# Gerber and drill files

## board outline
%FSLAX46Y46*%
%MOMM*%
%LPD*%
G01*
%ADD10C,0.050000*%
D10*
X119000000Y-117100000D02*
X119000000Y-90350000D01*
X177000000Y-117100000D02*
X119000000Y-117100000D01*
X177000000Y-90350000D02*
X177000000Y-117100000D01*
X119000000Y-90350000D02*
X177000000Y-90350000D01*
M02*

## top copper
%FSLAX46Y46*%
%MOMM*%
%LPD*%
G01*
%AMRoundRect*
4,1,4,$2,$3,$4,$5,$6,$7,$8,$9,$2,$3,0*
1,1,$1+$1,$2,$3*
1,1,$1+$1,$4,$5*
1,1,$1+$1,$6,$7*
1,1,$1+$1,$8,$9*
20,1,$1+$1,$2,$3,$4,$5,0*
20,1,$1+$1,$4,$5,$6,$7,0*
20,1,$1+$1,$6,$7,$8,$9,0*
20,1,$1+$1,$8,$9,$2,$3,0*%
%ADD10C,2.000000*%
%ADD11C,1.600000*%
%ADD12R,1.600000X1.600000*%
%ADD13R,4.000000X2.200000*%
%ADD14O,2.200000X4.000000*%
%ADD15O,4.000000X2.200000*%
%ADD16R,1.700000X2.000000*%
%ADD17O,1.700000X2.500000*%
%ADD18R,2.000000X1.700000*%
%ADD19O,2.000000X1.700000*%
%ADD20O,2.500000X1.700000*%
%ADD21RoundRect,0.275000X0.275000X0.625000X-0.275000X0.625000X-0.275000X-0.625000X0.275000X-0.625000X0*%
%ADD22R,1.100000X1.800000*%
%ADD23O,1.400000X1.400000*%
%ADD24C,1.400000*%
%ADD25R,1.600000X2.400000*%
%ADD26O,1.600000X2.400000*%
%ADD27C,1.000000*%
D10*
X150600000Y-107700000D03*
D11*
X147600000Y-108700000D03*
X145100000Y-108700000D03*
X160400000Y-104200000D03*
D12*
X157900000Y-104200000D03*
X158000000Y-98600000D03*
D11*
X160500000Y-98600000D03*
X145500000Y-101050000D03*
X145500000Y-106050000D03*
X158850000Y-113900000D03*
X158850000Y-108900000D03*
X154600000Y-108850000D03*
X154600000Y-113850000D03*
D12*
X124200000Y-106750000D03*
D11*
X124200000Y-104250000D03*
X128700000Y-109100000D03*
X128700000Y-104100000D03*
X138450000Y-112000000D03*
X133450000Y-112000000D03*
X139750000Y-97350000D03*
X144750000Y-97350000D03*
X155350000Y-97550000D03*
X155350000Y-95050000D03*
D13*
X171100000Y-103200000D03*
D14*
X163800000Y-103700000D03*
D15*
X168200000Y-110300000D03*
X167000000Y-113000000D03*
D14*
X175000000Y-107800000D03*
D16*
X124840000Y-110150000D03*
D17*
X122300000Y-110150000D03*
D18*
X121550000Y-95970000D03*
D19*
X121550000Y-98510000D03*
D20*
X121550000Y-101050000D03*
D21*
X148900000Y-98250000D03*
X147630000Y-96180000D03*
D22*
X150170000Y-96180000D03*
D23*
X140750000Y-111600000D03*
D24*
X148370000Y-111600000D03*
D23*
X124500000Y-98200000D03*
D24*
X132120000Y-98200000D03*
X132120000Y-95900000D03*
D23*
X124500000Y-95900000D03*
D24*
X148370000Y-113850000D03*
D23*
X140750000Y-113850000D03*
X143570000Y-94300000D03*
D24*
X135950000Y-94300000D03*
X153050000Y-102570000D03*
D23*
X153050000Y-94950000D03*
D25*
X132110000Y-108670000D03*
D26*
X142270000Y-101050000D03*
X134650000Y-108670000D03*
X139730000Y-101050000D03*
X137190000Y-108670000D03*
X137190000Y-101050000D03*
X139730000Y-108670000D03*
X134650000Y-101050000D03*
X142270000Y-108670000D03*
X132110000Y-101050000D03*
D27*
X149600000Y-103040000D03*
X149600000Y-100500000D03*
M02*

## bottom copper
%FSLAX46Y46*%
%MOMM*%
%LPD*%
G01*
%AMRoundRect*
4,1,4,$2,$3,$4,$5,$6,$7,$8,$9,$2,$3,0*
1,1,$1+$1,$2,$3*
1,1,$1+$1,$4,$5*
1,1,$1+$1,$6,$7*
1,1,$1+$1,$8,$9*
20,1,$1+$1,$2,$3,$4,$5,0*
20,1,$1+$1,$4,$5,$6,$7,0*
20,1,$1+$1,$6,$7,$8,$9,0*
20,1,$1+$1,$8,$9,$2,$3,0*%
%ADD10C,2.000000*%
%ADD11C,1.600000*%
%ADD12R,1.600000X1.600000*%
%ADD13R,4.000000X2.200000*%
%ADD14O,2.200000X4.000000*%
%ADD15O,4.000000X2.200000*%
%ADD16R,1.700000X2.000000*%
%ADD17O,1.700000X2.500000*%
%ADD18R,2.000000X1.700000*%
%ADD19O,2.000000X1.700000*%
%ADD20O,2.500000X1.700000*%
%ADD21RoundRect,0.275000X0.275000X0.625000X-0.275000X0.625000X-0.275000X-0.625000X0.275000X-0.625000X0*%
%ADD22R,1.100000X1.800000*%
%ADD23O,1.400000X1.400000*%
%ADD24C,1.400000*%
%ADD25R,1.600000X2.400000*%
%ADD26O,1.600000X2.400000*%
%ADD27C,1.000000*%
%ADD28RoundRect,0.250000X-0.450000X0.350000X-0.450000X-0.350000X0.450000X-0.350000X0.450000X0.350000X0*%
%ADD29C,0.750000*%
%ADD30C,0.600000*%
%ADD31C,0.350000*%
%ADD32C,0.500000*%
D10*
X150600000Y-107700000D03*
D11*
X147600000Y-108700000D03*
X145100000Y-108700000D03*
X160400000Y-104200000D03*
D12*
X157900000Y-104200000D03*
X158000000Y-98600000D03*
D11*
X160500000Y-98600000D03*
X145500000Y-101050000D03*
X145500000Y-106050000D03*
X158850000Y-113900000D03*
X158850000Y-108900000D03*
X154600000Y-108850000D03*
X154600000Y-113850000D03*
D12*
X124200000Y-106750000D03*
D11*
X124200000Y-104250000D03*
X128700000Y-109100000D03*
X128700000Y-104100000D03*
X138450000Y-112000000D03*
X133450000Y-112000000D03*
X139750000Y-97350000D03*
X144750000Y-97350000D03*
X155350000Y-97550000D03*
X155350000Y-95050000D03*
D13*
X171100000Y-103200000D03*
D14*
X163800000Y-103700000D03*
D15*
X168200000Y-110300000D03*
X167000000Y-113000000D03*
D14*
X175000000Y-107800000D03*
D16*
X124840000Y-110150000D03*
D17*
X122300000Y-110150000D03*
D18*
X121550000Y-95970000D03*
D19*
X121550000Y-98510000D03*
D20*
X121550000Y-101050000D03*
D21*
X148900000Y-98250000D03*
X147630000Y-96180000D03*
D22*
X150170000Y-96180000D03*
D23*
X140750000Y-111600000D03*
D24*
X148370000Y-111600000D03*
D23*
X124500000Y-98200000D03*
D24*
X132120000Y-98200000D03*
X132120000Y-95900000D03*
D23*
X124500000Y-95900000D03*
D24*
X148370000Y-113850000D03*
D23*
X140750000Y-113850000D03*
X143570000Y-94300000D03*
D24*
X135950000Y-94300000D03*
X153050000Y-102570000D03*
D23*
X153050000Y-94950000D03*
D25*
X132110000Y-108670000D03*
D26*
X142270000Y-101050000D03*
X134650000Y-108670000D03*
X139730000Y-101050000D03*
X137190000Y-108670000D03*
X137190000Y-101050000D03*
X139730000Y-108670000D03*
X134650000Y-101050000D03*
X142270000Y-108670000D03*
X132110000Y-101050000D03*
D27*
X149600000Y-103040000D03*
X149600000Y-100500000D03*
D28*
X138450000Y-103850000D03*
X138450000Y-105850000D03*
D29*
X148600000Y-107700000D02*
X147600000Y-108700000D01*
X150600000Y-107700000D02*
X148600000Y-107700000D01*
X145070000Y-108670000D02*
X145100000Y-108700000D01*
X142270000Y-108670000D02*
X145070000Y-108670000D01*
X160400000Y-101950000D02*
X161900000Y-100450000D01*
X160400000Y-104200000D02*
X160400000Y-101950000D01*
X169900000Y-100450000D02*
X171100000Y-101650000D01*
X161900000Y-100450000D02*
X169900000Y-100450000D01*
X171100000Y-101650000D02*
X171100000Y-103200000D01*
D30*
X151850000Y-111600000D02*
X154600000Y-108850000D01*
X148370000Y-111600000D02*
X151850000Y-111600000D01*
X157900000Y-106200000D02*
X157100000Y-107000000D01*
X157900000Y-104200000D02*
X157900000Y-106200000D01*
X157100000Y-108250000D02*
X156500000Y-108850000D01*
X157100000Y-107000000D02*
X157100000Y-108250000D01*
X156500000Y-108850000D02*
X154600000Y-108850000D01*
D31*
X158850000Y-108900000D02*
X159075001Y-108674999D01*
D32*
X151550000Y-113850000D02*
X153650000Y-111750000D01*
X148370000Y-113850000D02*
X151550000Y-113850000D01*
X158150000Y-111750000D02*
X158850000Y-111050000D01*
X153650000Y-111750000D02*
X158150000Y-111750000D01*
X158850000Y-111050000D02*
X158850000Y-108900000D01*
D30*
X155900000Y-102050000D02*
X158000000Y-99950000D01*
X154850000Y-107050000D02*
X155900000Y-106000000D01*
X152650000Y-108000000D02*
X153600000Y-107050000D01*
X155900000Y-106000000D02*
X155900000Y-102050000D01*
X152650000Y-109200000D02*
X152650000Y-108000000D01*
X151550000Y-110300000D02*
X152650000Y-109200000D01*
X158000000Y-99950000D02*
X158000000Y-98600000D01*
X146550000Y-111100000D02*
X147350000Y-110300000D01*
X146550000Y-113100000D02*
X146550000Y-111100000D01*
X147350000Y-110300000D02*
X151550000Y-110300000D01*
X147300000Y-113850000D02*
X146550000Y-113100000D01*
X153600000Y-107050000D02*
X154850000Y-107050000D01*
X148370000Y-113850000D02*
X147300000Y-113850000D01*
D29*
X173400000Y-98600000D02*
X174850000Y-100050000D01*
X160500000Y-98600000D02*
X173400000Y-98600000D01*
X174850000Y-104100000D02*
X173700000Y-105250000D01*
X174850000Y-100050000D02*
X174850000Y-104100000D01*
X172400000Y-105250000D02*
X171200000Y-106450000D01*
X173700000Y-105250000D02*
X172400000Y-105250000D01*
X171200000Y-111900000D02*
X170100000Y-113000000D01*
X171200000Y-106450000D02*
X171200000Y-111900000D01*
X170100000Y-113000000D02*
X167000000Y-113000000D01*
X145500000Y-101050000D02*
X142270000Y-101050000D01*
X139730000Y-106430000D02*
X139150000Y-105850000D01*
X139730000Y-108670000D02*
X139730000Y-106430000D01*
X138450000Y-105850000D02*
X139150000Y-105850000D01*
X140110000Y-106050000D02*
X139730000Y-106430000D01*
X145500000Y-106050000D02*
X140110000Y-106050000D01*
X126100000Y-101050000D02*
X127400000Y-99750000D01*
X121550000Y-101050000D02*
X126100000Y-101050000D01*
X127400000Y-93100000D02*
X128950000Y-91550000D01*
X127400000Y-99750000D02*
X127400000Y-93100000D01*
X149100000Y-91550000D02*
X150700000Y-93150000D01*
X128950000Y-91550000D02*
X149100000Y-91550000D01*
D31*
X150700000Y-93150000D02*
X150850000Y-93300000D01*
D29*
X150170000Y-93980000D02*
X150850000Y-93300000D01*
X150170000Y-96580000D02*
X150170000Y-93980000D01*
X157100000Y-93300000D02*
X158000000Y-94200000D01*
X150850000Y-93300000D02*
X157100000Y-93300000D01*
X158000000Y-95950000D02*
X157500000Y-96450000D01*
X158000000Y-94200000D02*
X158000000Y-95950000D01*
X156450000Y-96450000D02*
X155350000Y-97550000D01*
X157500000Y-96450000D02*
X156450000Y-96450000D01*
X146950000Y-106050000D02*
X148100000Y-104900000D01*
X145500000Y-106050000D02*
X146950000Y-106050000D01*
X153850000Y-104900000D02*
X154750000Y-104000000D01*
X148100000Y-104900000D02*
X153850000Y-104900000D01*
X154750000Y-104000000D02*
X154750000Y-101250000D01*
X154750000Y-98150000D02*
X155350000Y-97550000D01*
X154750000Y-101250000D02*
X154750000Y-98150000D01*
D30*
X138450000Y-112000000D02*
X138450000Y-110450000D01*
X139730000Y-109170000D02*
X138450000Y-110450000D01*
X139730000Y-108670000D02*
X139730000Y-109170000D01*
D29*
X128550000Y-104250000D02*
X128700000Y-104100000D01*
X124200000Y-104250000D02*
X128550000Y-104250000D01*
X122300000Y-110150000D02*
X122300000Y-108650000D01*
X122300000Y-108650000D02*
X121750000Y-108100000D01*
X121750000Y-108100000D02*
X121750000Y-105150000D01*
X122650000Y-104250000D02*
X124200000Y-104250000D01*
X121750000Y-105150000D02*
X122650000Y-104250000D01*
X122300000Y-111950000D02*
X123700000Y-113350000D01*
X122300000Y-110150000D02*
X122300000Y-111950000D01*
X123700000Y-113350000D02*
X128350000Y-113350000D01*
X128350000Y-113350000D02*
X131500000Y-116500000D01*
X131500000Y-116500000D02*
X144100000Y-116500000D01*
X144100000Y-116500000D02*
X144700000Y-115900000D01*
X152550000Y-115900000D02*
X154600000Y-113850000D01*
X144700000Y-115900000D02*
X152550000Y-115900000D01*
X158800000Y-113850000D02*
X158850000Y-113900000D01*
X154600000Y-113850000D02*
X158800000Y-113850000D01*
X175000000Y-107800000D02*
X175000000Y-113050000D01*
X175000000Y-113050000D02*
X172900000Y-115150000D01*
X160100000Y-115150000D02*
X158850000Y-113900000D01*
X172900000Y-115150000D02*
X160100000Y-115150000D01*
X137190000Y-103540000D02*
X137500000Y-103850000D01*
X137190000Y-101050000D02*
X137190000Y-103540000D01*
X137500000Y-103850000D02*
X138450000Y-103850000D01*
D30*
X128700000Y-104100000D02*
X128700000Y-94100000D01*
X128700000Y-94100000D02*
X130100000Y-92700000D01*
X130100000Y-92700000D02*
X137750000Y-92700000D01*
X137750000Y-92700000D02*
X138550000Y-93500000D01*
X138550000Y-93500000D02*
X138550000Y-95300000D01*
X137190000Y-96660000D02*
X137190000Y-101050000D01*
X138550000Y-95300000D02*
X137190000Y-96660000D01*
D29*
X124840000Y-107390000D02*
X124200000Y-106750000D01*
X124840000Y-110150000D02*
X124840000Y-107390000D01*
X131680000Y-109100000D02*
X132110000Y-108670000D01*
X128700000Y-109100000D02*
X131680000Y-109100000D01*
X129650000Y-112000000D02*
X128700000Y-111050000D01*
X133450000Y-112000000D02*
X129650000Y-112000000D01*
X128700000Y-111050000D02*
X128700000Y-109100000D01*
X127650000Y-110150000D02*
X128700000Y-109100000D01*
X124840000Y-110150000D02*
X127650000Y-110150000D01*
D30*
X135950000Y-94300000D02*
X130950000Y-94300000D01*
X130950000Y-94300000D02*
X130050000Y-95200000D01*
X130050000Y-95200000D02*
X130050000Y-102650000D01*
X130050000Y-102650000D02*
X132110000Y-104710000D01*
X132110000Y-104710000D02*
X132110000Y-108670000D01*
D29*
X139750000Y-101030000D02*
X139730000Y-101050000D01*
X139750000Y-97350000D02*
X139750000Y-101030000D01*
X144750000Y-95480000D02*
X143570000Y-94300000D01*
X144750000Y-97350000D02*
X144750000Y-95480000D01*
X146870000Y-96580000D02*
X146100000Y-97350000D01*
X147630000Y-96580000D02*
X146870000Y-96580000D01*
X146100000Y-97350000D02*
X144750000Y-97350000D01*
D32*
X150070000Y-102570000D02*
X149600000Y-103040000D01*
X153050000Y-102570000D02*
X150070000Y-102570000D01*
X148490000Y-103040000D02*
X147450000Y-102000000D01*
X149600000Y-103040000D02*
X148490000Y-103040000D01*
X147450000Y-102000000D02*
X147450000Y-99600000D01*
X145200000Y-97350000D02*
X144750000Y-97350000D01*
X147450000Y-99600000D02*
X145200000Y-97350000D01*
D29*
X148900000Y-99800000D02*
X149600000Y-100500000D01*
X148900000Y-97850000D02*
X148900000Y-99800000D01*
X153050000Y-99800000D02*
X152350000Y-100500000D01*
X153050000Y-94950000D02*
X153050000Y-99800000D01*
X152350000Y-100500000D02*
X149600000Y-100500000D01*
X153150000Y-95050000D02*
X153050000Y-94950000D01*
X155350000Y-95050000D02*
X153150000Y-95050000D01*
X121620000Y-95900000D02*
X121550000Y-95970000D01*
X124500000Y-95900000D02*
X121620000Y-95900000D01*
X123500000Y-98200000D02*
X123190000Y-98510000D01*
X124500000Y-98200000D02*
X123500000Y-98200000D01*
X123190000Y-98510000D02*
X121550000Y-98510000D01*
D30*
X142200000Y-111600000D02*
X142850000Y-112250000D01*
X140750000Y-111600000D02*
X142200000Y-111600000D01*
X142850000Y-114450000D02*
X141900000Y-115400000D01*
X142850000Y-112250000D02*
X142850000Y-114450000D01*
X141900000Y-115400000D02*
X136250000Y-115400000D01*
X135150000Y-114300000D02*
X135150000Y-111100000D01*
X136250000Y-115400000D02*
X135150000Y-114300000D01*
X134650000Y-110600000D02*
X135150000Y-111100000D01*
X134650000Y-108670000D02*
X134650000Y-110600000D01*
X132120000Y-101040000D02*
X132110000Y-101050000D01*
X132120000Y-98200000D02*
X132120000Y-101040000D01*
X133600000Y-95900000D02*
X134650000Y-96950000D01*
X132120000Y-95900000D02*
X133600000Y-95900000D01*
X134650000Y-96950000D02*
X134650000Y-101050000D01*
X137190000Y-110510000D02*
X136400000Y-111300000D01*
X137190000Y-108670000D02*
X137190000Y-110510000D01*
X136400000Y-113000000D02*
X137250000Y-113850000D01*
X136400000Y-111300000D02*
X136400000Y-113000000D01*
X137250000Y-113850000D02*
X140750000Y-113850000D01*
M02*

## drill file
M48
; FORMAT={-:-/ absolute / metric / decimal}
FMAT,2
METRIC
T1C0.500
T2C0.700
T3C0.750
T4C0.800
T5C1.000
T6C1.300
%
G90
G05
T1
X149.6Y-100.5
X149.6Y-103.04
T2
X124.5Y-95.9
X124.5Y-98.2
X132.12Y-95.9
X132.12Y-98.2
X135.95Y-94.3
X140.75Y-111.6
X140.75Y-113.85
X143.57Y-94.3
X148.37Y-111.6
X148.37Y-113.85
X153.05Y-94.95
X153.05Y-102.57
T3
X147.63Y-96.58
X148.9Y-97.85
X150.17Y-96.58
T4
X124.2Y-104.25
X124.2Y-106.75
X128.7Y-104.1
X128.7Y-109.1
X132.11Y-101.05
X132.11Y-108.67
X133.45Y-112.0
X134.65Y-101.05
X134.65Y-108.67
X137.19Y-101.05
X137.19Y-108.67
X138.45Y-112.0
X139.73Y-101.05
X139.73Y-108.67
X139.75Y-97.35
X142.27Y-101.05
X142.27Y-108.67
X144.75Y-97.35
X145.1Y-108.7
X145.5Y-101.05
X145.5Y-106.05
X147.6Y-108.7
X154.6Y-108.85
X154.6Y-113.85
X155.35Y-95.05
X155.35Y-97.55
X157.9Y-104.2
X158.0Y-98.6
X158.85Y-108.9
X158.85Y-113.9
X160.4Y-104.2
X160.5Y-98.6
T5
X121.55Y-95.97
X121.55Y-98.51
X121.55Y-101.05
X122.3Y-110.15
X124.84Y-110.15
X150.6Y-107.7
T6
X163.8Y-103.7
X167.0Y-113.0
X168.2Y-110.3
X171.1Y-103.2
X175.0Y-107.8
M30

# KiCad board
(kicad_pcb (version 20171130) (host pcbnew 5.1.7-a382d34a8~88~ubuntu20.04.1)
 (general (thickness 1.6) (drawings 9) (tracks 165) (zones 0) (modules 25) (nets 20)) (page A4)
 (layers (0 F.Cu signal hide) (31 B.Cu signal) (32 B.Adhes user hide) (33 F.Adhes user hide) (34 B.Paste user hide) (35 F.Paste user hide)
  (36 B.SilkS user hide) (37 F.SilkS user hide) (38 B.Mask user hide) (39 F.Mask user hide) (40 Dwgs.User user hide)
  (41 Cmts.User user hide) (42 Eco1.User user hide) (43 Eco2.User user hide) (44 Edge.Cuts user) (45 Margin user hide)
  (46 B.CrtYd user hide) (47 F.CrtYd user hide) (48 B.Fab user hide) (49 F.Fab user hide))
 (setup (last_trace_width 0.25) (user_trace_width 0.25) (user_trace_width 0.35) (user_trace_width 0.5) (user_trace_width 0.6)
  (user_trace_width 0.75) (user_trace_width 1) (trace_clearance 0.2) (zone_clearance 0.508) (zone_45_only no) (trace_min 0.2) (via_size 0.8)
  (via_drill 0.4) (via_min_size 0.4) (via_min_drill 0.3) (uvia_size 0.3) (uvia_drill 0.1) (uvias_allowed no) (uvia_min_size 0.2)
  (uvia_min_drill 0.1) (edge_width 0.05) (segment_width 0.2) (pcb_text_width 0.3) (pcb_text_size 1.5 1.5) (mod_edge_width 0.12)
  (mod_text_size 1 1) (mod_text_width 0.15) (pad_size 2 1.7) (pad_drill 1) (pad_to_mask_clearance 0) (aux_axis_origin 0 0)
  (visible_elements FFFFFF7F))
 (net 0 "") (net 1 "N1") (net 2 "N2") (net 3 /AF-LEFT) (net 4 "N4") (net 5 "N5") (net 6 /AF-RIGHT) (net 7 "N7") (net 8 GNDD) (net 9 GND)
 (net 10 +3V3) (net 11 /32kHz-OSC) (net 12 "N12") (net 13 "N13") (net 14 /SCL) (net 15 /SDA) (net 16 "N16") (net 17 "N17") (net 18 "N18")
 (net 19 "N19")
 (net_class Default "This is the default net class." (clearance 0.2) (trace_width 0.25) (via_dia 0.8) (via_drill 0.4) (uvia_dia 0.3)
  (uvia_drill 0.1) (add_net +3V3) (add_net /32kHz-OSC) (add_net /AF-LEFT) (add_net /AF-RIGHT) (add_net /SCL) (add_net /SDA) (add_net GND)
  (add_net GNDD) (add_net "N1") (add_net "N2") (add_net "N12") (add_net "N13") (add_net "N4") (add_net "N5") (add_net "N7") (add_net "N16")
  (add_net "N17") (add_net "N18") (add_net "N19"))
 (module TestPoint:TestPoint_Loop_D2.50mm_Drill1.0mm (layer F.Cu) (at 150.6 107.7)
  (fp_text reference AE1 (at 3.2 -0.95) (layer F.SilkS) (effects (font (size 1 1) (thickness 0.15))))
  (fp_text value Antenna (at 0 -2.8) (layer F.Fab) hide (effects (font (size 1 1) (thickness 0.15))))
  (pad 1 thru_hole circle (at 0 0) (size 2 2) (drill 1) (layers *.Cu *.Mask) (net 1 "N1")))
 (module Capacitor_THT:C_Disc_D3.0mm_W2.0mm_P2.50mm (layer F.Cu) (at 147.6 108.7 180)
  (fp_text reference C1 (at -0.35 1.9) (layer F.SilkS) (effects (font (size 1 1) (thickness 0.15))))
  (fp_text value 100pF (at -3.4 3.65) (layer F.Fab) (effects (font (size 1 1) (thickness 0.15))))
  (pad 1 thru_hole circle (at 0 0 180) (size 1.6 1.6) (drill 0.8) (layers *.Cu *.Mask) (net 1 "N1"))
  (pad 2 thru_hole circle (at 2.5 0 180) (size 1.6 1.6) (drill 0.8) (layers *.Cu *.Mask) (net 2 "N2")))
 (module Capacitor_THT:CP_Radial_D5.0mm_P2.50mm (layer F.Cu) (at 157.9 104.2)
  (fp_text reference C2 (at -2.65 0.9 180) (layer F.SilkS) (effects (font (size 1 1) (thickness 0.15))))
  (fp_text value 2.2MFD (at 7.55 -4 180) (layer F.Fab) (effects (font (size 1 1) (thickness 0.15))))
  (pad 2 thru_hole circle (at 2.5 0) (size 1.6 1.6) (drill 0.8) (layers *.Cu *.Mask) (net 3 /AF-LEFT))
  (pad 1 thru_hole rect (at 0 0) (size 1.6 1.6) (drill 0.8) (layers *.Cu *.Mask) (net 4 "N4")))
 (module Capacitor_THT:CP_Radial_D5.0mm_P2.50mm (layer F.Cu) (at 158 98.6)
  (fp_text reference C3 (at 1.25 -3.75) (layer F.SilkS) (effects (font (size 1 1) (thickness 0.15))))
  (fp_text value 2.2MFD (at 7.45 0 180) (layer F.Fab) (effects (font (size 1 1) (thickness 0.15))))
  (pad 1 thru_hole rect (at 0 0) (size 1.6 1.6) (drill 0.8) (layers *.Cu *.Mask) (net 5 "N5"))
  (pad 2 thru_hole circle (at 2.5 0) (size 1.6 1.6) (drill 0.8) (layers *.Cu *.Mask) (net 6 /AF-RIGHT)))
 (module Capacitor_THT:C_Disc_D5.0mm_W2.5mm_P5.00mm (layer F.Cu) (at 145.5 101.05 270)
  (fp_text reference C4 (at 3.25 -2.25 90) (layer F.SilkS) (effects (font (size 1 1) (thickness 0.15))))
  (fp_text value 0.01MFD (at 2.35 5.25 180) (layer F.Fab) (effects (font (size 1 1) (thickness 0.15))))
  (pad 1 thru_hole circle (at 0 0 270) (size 1.6 1.6) (drill 0.8) (layers *.Cu *.Mask) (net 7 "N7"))
  (pad 2 thru_hole circle (at 5 0 270) (size 1.6 1.6) (drill 0.8) (layers *.Cu *.Mask) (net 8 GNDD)))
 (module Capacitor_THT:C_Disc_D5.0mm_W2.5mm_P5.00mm (layer F.Cu) (at 158.85 108.9 270)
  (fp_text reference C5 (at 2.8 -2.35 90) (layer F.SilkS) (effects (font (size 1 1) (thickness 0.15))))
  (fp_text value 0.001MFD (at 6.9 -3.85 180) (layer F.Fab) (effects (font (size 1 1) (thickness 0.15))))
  (pad 2 thru_hole circle (at 5 0 270) (size 1.6 1.6) (drill 0.8) (layers *.Cu *.Mask) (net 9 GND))
  (pad 1 thru_hole circle (at 0 0 270) (size 1.6 1.6) (drill 0.8) (layers *.Cu *.Mask) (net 5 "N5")))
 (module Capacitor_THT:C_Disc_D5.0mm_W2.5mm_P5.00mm (layer F.Cu) (at 154.6 108.85 270)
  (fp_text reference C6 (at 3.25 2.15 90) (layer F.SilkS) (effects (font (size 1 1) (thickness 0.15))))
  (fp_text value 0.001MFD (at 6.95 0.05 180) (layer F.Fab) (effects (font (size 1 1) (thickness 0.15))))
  (pad 1 thru_hole circle (at 0 0 270) (size 1.6 1.6) (drill 0.8) (layers *.Cu *.Mask) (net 4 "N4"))
  (pad 2 thru_hole circle (at 5 0 270) (size 1.6 1.6) (drill 0.8) (layers *.Cu *.Mask) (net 9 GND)))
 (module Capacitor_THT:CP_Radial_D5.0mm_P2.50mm (layer F.Cu) (at 124.2 106.75 90)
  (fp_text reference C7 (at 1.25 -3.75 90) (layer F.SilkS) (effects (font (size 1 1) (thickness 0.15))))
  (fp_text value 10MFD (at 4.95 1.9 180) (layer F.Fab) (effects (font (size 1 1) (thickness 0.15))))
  (pad 1 thru_hole rect (at 0 0 90) (size 1.6 1.6) (drill 0.8) (layers *.Cu *.Mask) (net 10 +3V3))
  (pad 2 thru_hole circle (at 2.5 0 90) (size 1.6 1.6) (drill 0.8) (layers *.Cu *.Mask) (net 9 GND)))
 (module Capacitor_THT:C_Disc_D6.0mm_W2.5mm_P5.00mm (layer F.Cu) (at 128.7 109.1 90)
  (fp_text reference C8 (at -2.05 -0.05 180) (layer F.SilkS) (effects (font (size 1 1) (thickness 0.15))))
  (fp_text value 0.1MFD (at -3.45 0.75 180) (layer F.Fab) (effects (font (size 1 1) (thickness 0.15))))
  (pad 1 thru_hole circle (at 0 0 90) (size 1.6 1.6) (drill 0.8) (layers *.Cu *.Mask) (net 10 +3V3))
  (pad 2 thru_hole circle (at 5 0 90) (size 1.6 1.6) (drill 0.8) (layers *.Cu *.Mask) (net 9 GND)))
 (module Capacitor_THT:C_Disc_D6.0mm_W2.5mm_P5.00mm (layer F.Cu) (at 133.45 112)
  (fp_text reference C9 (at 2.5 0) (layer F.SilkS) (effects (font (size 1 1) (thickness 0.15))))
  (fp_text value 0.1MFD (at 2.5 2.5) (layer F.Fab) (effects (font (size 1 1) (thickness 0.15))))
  (pad 2 thru_hole circle (at 5 0) (size 1.6 1.6) (drill 0.8) (layers *.Cu *.Mask) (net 8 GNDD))
  (pad 1 thru_hole circle (at 0 0) (size 1.6 1.6) (drill 0.8) (layers *.Cu *.Mask) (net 10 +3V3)))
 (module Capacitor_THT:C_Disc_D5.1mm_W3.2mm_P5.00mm (layer F.Cu) (at 139.75 97.35)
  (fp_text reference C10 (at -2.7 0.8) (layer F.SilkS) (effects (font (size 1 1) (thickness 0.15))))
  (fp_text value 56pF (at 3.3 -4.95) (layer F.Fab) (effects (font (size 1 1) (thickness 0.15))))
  (pad 1 thru_hole circle (at 0 0) (size 1.6 1.6) (drill 0.8) (layers *.Cu *.Mask) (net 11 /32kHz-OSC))
  (pad 2 thru_hole circle (at 5 0) (size 1.6 1.6) (drill 0.8) (layers *.Cu *.Mask) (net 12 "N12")))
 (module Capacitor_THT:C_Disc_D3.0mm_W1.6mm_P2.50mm (layer F.Cu) (at 155.35 97.55 90)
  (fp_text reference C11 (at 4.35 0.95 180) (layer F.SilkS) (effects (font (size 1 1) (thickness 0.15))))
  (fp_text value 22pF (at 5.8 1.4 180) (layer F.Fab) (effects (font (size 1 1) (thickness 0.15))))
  (pad 1 thru_hole circle (at 0 0 90) (size 1.6 1.6) (drill 0.8) (layers *.Cu *.Mask) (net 8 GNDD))
  (pad 2 thru_hole circle (at 2.5 0 90) (size 1.6 1.6) (drill 0.8) (layers *.Cu *.Mask) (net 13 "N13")))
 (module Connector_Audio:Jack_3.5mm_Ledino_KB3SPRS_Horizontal (layer F.Cu) (at 171.1 103.2 180)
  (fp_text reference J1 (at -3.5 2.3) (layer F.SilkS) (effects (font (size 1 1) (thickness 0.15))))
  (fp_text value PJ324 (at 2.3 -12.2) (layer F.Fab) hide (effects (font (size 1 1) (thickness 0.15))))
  (pad T thru_hole rect (at 0 0 180) (size 4 2.2) (drill 1.3) (layers *.Cu *.Mask) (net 3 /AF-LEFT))
  (pad TN thru_hole oval (at 7.3 -0.5 270) (size 4 2.2) (drill 1.3) (layers *.Cu *.Mask))
  (pad RN thru_hole oval (at 2.9 -7.1 180) (size 4 2.2) (drill 1.3) (layers *.Cu *.Mask))
  (pad R thru_hole oval (at 4.1 -9.8 180) (size 4 2.2) (drill 1.3) (layers *.Cu *.Mask) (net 6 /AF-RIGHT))
  (pad S thru_hole oval (at -3.9 -4.6 180) (size 2.2 4) (drill 1.3) (layers *.Cu *.Mask) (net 9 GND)))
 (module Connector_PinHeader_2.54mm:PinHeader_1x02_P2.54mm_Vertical (layer F.Cu) (at 124.84 110.15 270)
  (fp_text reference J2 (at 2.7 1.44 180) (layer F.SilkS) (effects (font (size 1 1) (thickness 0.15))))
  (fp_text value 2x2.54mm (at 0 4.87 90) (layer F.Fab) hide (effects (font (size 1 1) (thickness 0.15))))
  (pad 1 thru_hole rect (at 0 0 270) (size 2 1.7) (drill 1) (layers *.Cu *.Mask) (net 10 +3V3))
  (pad 2 thru_hole oval (at 0 2.54 270) (size 2.5 1.7) (drill 1) (layers *.Cu *.Mask) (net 9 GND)))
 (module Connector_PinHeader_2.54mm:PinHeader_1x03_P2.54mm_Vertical (layer F.Cu) (at 121.55 95.97)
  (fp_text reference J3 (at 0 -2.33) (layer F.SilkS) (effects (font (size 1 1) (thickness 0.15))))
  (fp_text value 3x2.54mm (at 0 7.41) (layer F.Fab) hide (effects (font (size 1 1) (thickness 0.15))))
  (pad 1 thru_hole rect (at 0 0) (size 2 1.7) (drill 1) (layers *.Cu *.Mask) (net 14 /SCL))
  (pad 2 thru_hole oval (at 0 2.54) (size 2 1.7) (drill 1) (layers *.Cu *.Mask) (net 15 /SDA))
  (pad 3 thru_hole oval (at 0 5.08) (size 2.5 1.7) (drill 1) (layers *.Cu *.Mask) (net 8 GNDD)))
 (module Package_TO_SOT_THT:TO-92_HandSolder (layer F.Cu) (at 150.17 96.58 180)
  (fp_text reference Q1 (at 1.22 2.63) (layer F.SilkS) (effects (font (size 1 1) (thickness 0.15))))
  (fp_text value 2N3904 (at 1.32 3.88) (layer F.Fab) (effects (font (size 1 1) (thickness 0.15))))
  (pad 2 thru_hole roundrect (at 1.27 -1.27 180) (size 1.1 1.8) (drill 0.75 (offset 0 -0.4)) (layers *.Cu *.Mask) (roundrect_rratio 0.25)
   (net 13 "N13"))
  (pad 3 thru_hole roundrect (at 2.54 0 180) (size 1.1 1.8) (drill 0.75 (offset 0 0.4)) (layers *.Cu *.Mask) (roundrect_rratio 0.25)
   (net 12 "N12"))
  (pad 1 thru_hole rect (at 0 0 180) (size 1.1 1.8) (drill 0.75 (offset 0 0.4)) (layers *.Cu *.Mask) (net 8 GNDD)))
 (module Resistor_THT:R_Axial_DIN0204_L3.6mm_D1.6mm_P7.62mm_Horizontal (layer F.Cu) (at 148.37 111.6 180)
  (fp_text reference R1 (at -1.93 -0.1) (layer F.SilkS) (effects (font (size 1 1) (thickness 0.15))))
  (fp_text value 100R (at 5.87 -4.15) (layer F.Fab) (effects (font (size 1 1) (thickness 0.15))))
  (pad 2 thru_hole oval (at 7.62 0 180) (size 1.4 1.4) (drill 0.7) (layers *.Cu *.Mask) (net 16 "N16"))
  (pad 1 thru_hole circle (at 0 0 180) (size 1.4 1.4) (drill 0.7) (layers *.Cu *.Mask) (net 4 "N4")))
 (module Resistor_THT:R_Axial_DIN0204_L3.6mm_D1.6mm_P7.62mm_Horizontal (layer F.Cu) (at 132.12 98.2 180)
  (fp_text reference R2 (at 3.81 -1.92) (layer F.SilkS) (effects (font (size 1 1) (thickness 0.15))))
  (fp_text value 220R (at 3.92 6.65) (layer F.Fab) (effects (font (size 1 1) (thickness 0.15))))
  (pad 2 thru_hole oval (at 7.62 0 180) (size 1.4 1.4) (drill 0.7) (layers *.Cu *.Mask) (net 15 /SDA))
  (pad 1 thru_hole circle (at 0 0 180) (size 1.4 1.4) (drill 0.7) (layers *.Cu *.Mask) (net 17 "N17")))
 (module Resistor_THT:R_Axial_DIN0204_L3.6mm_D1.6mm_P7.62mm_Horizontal (layer F.Cu) (at 132.12 95.9 180)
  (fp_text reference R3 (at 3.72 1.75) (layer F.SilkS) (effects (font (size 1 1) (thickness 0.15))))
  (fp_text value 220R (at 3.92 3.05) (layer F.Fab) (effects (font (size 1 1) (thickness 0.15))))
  (pad 1 thru_hole circle (at 0 0 180) (size 1.4 1.4) (drill 0.7) (layers *.Cu *.Mask) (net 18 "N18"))
  (pad 2 thru_hole oval (at 7.62 0 180) (size 1.4 1.4) (drill 0.7) (layers *.Cu *.Mask) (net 14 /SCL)))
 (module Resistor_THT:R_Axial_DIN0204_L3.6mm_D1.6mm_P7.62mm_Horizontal (layer F.Cu) (at 148.37 113.85 180)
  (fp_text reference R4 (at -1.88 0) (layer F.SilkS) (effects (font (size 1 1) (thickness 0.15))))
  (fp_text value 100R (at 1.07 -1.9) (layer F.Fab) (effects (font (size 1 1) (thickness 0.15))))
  (pad 1 thru_hole circle (at 0 0 180) (size 1.4 1.4) (drill 0.7) (layers *.Cu *.Mask) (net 5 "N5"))
  (pad 2 thru_hole oval (at 7.62 0 180) (size 1.4 1.4) (drill 0.7) (layers *.Cu *.Mask) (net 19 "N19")))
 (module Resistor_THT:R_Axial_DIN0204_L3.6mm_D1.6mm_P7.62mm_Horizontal (layer F.Cu) (at 135.95 94.3)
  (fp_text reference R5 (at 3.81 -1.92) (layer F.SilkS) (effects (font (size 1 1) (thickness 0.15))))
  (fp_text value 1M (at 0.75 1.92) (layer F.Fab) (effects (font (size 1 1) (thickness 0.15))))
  (pad 2 thru_hole oval (at 7.62 0) (size 1.4 1.4) (drill 0.7) (layers *.Cu *.Mask) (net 12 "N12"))
  (pad 1 thru_hole circle (at 0 0) (size 1.4 1.4) (drill 0.7) (layers *.Cu *.Mask) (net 10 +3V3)))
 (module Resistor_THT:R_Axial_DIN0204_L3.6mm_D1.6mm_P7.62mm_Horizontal (layer F.Cu) (at 153.05 102.57 90)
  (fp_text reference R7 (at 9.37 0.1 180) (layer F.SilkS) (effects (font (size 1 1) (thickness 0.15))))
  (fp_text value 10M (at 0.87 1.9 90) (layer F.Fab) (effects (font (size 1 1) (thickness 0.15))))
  (pad 1 thru_hole circle (at 0 0 90) (size 1.4 1.4) (drill 0.7) (layers *.Cu *.Mask) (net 12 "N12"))
  (pad 2 thru_hole oval (at 7.62 0 90) (size 1.4 1.4) (drill 0.7) (layers *.Cu *.Mask) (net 13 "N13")))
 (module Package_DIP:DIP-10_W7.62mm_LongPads (layer F.Cu) (at 132.11 108.67 90)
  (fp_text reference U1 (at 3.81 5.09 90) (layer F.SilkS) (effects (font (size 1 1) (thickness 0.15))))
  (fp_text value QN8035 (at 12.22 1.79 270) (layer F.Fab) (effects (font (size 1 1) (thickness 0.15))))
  (pad 1 thru_hole rect (at 0 0 90) (size 2.4 1.6) (drill 0.8) (layers *.Cu *.Mask) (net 10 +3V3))
  (pad 6 thru_hole oval (at 7.62 10.16 90) (size 2.4 1.6) (drill 0.8) (layers *.Cu *.Mask) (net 7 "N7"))
  (pad 2 thru_hole oval (at 0 2.54 90) (size 2.4 1.6) (drill 0.8) (layers *.Cu *.Mask) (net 16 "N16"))
  (pad 7 thru_hole oval (at 7.62 7.62 90) (size 2.4 1.6) (drill 0.8) (layers *.Cu *.Mask) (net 11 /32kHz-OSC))
  (pad 3 thru_hole oval (at 0 5.08 90) (size 2.4 1.6) (drill 0.8) (layers *.Cu *.Mask) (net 19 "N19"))
  (pad 8 thru_hole oval (at 7.62 5.08 90) (size 2.4 1.6) (drill 0.8) (layers *.Cu *.Mask) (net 9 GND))
  (pad 4 thru_hole oval (at 0 7.62 90) (size 2.4 1.6) (drill 0.8) (layers *.Cu *.Mask) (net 8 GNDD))
  (pad 9 thru_hole oval (at 7.62 2.54 90) (size 2.4 1.6) (drill 0.8) (layers *.Cu *.Mask) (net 18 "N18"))
  (pad 5 thru_hole oval (at 0 10.16 90) (size 2.4 1.6) (drill 0.8) (layers *.Cu *.Mask) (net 2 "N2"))
  (pad 10 thru_hole oval (at 7.62 0 90) (size 2.4 1.6) (drill 0.8) (layers *.Cu *.Mask) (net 17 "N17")))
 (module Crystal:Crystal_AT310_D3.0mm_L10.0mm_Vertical (layer F.Cu) (at 149.6 103.04 90)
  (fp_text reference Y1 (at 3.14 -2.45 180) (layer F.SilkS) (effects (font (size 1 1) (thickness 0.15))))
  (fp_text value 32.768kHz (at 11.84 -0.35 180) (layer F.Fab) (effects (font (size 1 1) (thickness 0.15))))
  (pad 1 thru_hole circle (at 0 0 90) (size 1 1) (drill 0.5) (layers *.Cu *.Mask) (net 12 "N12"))
  (pad 2 thru_hole circle (at 2.54 0 90) (size 1 1) (drill 0.5) (layers *.Cu *.Mask) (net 13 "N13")))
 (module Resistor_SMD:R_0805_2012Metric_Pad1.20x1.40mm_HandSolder (layer B.Cu) (at 138.45 104.85 270)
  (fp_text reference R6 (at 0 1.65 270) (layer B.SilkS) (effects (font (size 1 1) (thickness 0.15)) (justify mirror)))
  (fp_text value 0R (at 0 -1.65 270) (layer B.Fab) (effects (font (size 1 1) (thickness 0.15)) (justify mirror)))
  (pad 1 smd roundrect (at -1 0 270) (size 1.2 1.4) (layers B.Cu B.Paste B.Mask) (roundrect_rratio 0.208333) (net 9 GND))
  (pad 2 smd roundrect (at 1 0 270) (size 1.2 1.4) (layers B.Cu B.Paste B.Mask) (roundrect_rratio 0.208333) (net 8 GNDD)))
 (gr_line (start 119 117.1) (end 119 90.35) (layer Edge.Cuts) (width 0.05))
 (gr_line (start 177 117.1) (end 119 117.1) (layer Edge.Cuts) (width 0.05))
 (gr_line (start 177 90.35) (end 177 117.1) (layer Edge.Cuts) (width 0.05))
 (gr_line (start 119 90.35) (end 177 90.35) (layer Edge.Cuts) (width 0.05))
 (segment (start 148.6 107.7) (end 147.6 108.7) (width 0.75) (layer B.Cu) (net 1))
 (segment (start 150.6 107.7) (end 148.6 107.7) (width 0.75) (layer B.Cu) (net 1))
 (segment (start 145.07 108.67) (end 145.1 108.7) (width 0.75) (layer B.Cu) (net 2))
 (segment (start 142.27 108.67) (end 145.07 108.67) (width 0.75) (layer B.Cu) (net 2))
 (segment (start 160.4 101.95) (end 161.9 100.45) (width 0.75) (layer B.Cu) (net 3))
 (segment (start 160.4 104.2) (end 160.4 101.95) (width 0.75) (layer B.Cu) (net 3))
 (segment (start 169.9 100.45) (end 171.1 101.65) (width 0.75) (layer B.Cu) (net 3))
 (segment (start 161.9 100.45) (end 169.9 100.45) (width 0.75) (layer B.Cu) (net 3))
 (segment (start 171.1 101.65) (end 171.1 103.2) (width 0.75) (layer B.Cu) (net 3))
 (segment (start 151.85 111.6) (end 154.6 108.85) (width 0.6) (layer B.Cu) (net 4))
 (segment (start 148.37 111.6) (end 151.85 111.6) (width 0.6) (layer B.Cu) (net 4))
 (segment (start 157.9 106.2) (end 157.1 107) (width 0.6) (layer B.Cu) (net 4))
 (segment (start 157.9 104.2) (end 157.9 106.2) (width 0.6) (layer B.Cu) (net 4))
 (segment (start 157.1 108.25) (end 156.5 108.85) (width 0.6) (layer B.Cu) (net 4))
 (segment (start 157.1 107) (end 157.1 108.25) (width 0.6) (layer B.Cu) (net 4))
 (segment (start 156.5 108.85) (end 154.6 108.85) (width 0.6) (layer B.Cu) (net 4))
 (segment (start 158.85 108.9) (end 159.075001 108.674999) (width 0.35) (layer B.Cu) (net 5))
 (segment (start 151.55 113.85) (end 153.65 111.75) (width 0.5) (layer B.Cu) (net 5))
 (segment (start 148.37 113.85) (end 151.55 113.85) (width 0.5) (layer B.Cu) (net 5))
 (segment (start 158.15 111.75) (end 158.85 111.05) (width 0.5) (layer B.Cu) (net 5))
 (segment (start 153.65 111.75) (end 158.15 111.75) (width 0.5) (layer B.Cu) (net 5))
 (segment (start 158.85 111.05) (end 158.85 108.9) (width 0.5) (layer B.Cu) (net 5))
 (segment (start 155.9 102.05) (end 158 99.95) (width 0.6) (layer B.Cu) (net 5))
 (segment (start 154.85 107.05) (end 155.9 106) (width 0.6) (layer B.Cu) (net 5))
 (segment (start 152.65 108) (end 153.6 107.05) (width 0.6) (layer B.Cu) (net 5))
 (segment (start 155.9 106) (end 155.9 102.05) (width 0.6) (layer B.Cu) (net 5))
 (segment (start 152.65 109.2) (end 152.65 108) (width 0.6) (layer B.Cu) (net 5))
 (segment (start 151.55 110.3) (end 152.65 109.2) (width 0.6) (layer B.Cu) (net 5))
 (segment (start 158 99.95) (end 158 98.6) (width 0.6) (layer B.Cu) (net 5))
 (segment (start 146.55 111.1) (end 147.35 110.3) (width 0.6) (layer B.Cu) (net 5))
 (segment (start 146.55 113.1) (end 146.55 111.1) (width 0.6) (layer B.Cu) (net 5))
 (segment (start 147.35 110.3) (end 151.55 110.3) (width 0.6) (layer B.Cu) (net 5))
 (segment (start 147.3 113.85) (end 146.55 113.1) (width 0.6) (layer B.Cu) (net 5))
 (segment (start 153.6 107.05) (end 154.85 107.05) (width 0.6) (layer B.Cu) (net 5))
 (segment (start 148.37 113.85) (end 147.3 113.85) (width 0.6) (layer B.Cu) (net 5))
 (segment (start 173.4 98.6) (end 174.85 100.05) (width 0.75) (layer B.Cu) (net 6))
 (segment (start 160.5 98.6) (end 173.4 98.6) (width 0.75) (layer B.Cu) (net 6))
 (segment (start 174.85 104.1) (end 173.7 105.25) (width 0.75) (layer B.Cu) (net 6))
 (segment (start 174.85 100.05) (end 174.85 104.1) (width 0.75) (layer B.Cu) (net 6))
 (segment (start 172.4 105.25) (end 171.2 106.45) (width 0.75) (layer B.Cu) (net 6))
 (segment (start 173.7 105.25) (end 172.4 105.25) (width 0.75) (layer B.Cu) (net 6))
 (segment (start 171.2 111.9) (end 170.1 113) (width 0.75) (layer B.Cu) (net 6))
 (segment (start 171.2 106.45) (end 171.2 111.9) (width 0.75) (layer B.Cu) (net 6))
 (segment (start 170.1 113) (end 167 113) (width 0.75) (layer B.Cu) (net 6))
 (segment (start 145.5 101.05) (end 142.27 101.05) (width 0.75) (layer B.Cu) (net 7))
 (segment (start 139.73 106.43) (end 139.15 105.85) (width 0.75) (layer B.Cu) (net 8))
 (segment (start 139.73 108.67) (end 139.73 106.43) (width 0.75) (layer B.Cu) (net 8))
 (segment (start 138.45 105.85) (end 139.15 105.85) (width 0.75) (layer B.Cu) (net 8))
 (segment (start 140.11 106.05) (end 139.73 106.43) (width 0.75) (layer B.Cu) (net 8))
 (segment (start 145.5 106.05) (end 140.11 106.05) (width 0.75) (layer B.Cu) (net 8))
 (segment (start 126.1 101.05) (end 127.4 99.75) (width 0.75) (layer B.Cu) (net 8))
 (segment (start 121.55 101.05) (end 126.1 101.05) (width 0.75) (layer B.Cu) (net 8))
 (segment (start 127.4 93.1) (end 128.95 91.55) (width 0.75) (layer B.Cu) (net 8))
 (segment (start 127.4 99.75) (end 127.4 93.1) (width 0.75) (layer B.Cu) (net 8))
 (segment (start 149.1 91.55) (end 150.7 93.15) (width 0.75) (layer B.Cu) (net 8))
 (segment (start 128.95 91.55) (end 149.1 91.55) (width 0.75) (layer B.Cu) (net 8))
 (segment (start 150.7 93.15) (end 150.85 93.3) (width 0.35) (layer B.Cu) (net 8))
 (segment (start 150.17 93.98) (end 150.85 93.3) (width 0.75) (layer B.Cu) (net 8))
 (segment (start 150.17 96.58) (end 150.17 93.98) (width 0.75) (layer B.Cu) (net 8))
 (segment (start 157.1 93.3) (end 158 94.2) (width 0.75) (layer B.Cu) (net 8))
 (segment (start 150.85 93.3) (end 157.1 93.3) (width 0.75) (layer B.Cu) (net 8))
 (segment (start 158 95.95) (end 157.5 96.45) (width 0.75) (layer B.Cu) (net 8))
 (segment (start 158 94.2) (end 158 95.95) (width 0.75) (layer B.Cu) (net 8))
 (segment (start 156.45 96.45) (end 155.35 97.55) (width 0.75) (layer B.Cu) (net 8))
 (segment (start 157.5 96.45) (end 156.45 96.45) (width 0.75) (layer B.Cu) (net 8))
 (segment (start 146.95 106.05) (end 148.1 104.9) (width 0.75) (layer B.Cu) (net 8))
 (segment (start 145.5 106.05) (end 146.95 106.05) (width 0.75) (layer B.Cu) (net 8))
 (segment (start 153.85 104.9) (end 154.75 104) (width 0.75) (layer B.Cu) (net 8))
 (segment (start 148.1 104.9) (end 153.85 104.9) (width 0.75) (layer B.Cu) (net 8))
 (segment (start 154.75 104) (end 154.75 101.25) (width 0.75) (layer B.Cu) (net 8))
 (segment (start 154.75 98.15) (end 155.35 97.55) (width 0.75) (layer B.Cu) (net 8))
 (segment (start 154.75 101.25) (end 154.75 98.15) (width 0.75) (layer B.Cu) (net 8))
 (segment (start 138.45 112) (end 138.45 110.45) (width 0.6) (layer B.Cu) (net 8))
 (segment (start 139.73 109.17) (end 138.45 110.45) (width 0.6) (layer B.Cu) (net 8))
 (segment (start 139.73 108.67) (end 139.73 109.17) (width 0.6) (layer B.Cu) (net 8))
 (segment (start 128.55 104.25) (end 128.7 104.1) (width 0.75) (layer B.Cu) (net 9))
 (segment (start 124.2 104.25) (end 128.55 104.25) (width 0.75) (layer B.Cu) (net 9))
 (segment (start 122.3 110.15) (end 122.3 108.65) (width 0.75) (layer B.Cu) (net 9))
 (segment (start 122.3 108.65) (end 121.75 108.1) (width 0.75) (layer B.Cu) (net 9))
 (segment (start 121.75 108.1) (end 121.75 105.15) (width 0.75) (layer B.Cu) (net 9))
 (segment (start 122.65 104.25) (end 124.2 104.25) (width 0.75) (layer B.Cu) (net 9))
 (segment (start 121.75 105.15) (end 122.65 104.25) (width 0.75) (layer B.Cu) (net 9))
 (segment (start 122.3 111.95) (end 123.7 113.35) (width 0.75) (layer B.Cu) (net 9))
 (segment (start 122.3 110.15) (end 122.3 111.95) (width 0.75) (layer B.Cu) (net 9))
 (segment (start 123.7 113.35) (end 128.35 113.35) (width 0.75) (layer B.Cu) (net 9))
 (segment (start 128.35 113.35) (end 131.5 116.5) (width 0.75) (layer B.Cu) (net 9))
 (segment (start 131.5 116.5) (end 144.1 116.5) (width 0.75) (layer B.Cu) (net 9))
 (segment (start 144.1 116.5) (end 144.7 115.9) (width 0.75) (layer B.Cu) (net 9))
 (segment (start 152.55 115.9) (end 154.6 113.85) (width 0.75) (layer B.Cu) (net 9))
 (segment (start 144.7 115.9) (end 152.55 115.9) (width 0.75) (layer B.Cu) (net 9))
 (segment (start 158.8 113.85) (end 158.85 113.9) (width 0.75) (layer B.Cu) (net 9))
 (segment (start 154.6 113.85) (end 158.8 113.85) (width 0.75) (layer B.Cu) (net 9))
 (segment (start 175 107.8) (end 175 113.05) (width 0.75) (layer B.Cu) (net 9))
 (segment (start 175 113.05) (end 172.9 115.15) (width 0.75) (layer B.Cu) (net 9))
 (segment (start 160.1 115.15) (end 158.85 113.9) (width 0.75) (layer B.Cu) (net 9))
 (segment (start 172.9 115.15) (end 160.1 115.15) (width 0.75) (layer B.Cu) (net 9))
 (segment (start 137.19 103.54) (end 137.5 103.85) (width 0.75) (layer B.Cu) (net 9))
 (segment (start 137.19 101.05) (end 137.19 103.54) (width 0.75) (layer B.Cu) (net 9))
 (segment (start 137.5 103.85) (end 138.45 103.85) (width 0.75) (layer B.Cu) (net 9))
 (segment (start 128.7 104.1) (end 128.7 94.1) (width 0.6) (layer B.Cu) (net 9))
 (segment (start 128.7 94.1) (end 130.1 92.7) (width 0.6) (layer B.Cu) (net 9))
 (segment (start 130.1 92.7) (end 137.75 92.7) (width 0.6) (layer B.Cu) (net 9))
 (segment (start 137.75 92.7) (end 138.55 93.5) (width 0.6) (layer B.Cu) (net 9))
 (segment (start 138.55 93.5) (end 138.55 95.3) (width 0.6) (layer B.Cu) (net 9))
 (segment (start 137.19 96.66) (end 137.19 101.05) (width 0.6) (layer B.Cu) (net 9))
 (segment (start 138.55 95.3) (end 137.19 96.66) (width 0.6) (layer B.Cu) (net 9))
 (segment (start 124.84 107.39) (end 124.2 106.75) (width 0.75) (layer B.Cu) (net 10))
 (segment (start 124.84 110.15) (end 124.84 107.39) (width 0.75) (layer B.Cu) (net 10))
 (segment (start 131.68 109.1) (end 132.11 108.67) (width 0.75) (layer B.Cu) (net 10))
 (segment (start 128.7 109.1) (end 131.68 109.1) (width 0.75) (layer B.Cu) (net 10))
 (segment (start 129.65 112) (end 128.7 111.05) (width 0.75) (layer B.Cu) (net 10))
 (segment (start 133.45 112) (end 129.65 112) (width 0.75) (layer B.Cu) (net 10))
 (segment (start 128.7 111.05) (end 128.7 109.1) (width 0.75) (layer B.Cu) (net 10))
 (segment (start 127.65 110.15) (end 128.7 109.1) (width 0.75) (layer B.Cu) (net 10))
 (segment (start 124.84 110.15) (end 127.65 110.15) (width 0.75) (layer B.Cu) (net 10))
 (segment (start 135.95 94.3) (end 130.95 94.3) (width 0.6) (layer B.Cu) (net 10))
 (segment (start 130.95 94.3) (end 130.05 95.2) (width 0.6) (layer B.Cu) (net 10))
 (segment (start 130.05 95.2) (end 130.05 102.65) (width 0.6) (layer B.Cu) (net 10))
 (segment (start 130.05 102.65) (end 132.11 104.71) (width 0.6) (layer B.Cu) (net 10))
 (segment (start 132.11 104.71) (end 132.11 108.67) (width 0.6) (layer B.Cu) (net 10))
 (segment (start 139.75 101.03) (end 139.73 101.05) (width 0.75) (layer B.Cu) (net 11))
 (segment (start 139.75 97.35) (end 139.75 101.03) (width 0.75) (layer B.Cu) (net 11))
 (segment (start 144.75 95.48) (end 143.57 94.3) (width 0.75) (layer B.Cu) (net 12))
 (segment (start 144.75 97.35) (end 144.75 95.48) (width 0.75) (layer B.Cu) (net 12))
 (segment (start 146.87 96.58) (end 146.1 97.35) (width 0.75) (layer B.Cu) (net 12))
 (segment (start 147.63 96.58) (end 146.87 96.58) (width 0.75) (layer B.Cu) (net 12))
 (segment (start 146.1 97.35) (end 144.75 97.35) (width 0.75) (layer B.Cu) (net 12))
 (segment (start 150.07 102.57) (end 149.6 103.04) (width 0.5) (layer B.Cu) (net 12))
 (segment (start 153.05 102.57) (end 150.07 102.57) (width 0.5) (layer B.Cu) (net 12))
 (segment (start 148.49 103.04) (end 147.45 102) (width 0.5) (layer B.Cu) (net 12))
 (segment (start 149.6 103.04) (end 148.49 103.04) (width 0.5) (layer B.Cu) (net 12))
 (segment (start 147.45 102) (end 147.45 99.6) (width 0.5) (layer B.Cu) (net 12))
 (segment (start 145.2 97.35) (end 144.75 97.35) (width 0.5) (layer B.Cu) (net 12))
 (segment (start 147.45 99.6) (end 145.2 97.35) (width 0.5) (layer B.Cu) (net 12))
 (segment (start 148.9 99.8) (end 149.6 100.5) (width 0.75) (layer B.Cu) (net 13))
 (segment (start 148.9 97.85) (end 148.9 99.8) (width 0.75) (layer B.Cu) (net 13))
 (segment (start 153.05 99.8) (end 152.35 100.5) (width 0.75) (layer B.Cu) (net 13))
 (segment (start 153.05 94.95) (end 153.05 99.8) (width 0.75) (layer B.Cu) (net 13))
 (segment (start 152.35 100.5) (end 149.6 100.5) (width 0.75) (layer B.Cu) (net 13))
 (segment (start 153.15 95.05) (end 153.05 94.95) (width 0.75) (layer B.Cu) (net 13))
 (segment (start 155.35 95.05) (end 153.15 95.05) (width 0.75) (layer B.Cu) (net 13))
 (segment (start 121.62 95.9) (end 121.55 95.97) (width 0.75) (layer B.Cu) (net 14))
 (segment (start 124.5 95.9) (end 121.62 95.9) (width 0.75) (layer B.Cu) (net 14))
 (segment (start 123.5 98.2) (end 123.19 98.51) (width 0.75) (layer B.Cu) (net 15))
 (segment (start 124.5 98.2) (end 123.5 98.2) (width 0.75) (layer B.Cu) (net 15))
 (segment (start 123.19 98.51) (end 121.55 98.51) (width 0.75) (layer B.Cu) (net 15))
 (segment (start 142.2 111.6) (end 142.85 112.25) (width 0.6) (layer B.Cu) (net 16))
 (segment (start 140.75 111.6) (end 142.2 111.6) (width 0.6) (layer B.Cu) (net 16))
 (segment (start 142.85 114.45) (end 141.9 115.4) (width 0.6) (layer B.Cu) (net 16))
 (segment (start 142.85 112.25) (end 142.85 114.45) (width 0.6) (layer B.Cu) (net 16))
 (segment (start 141.9 115.4) (end 136.25 115.4) (width 0.6) (layer B.Cu) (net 16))
 (segment (start 135.15 114.3) (end 135.15 111.1) (width 0.6) (layer B.Cu) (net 16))
 (segment (start 136.25 115.4) (end 135.15 114.3) (width 0.6) (layer B.Cu) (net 16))
 (segment (start 134.65 110.6) (end 135.15 111.1) (width 0.6) (layer B.Cu) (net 16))
 (segment (start 134.65 108.67) (end 134.65 110.6) (width 0.6) (layer B.Cu) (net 16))
 (segment (start 132.12 101.04) (end 132.11 101.05) (width 0.6) (layer B.Cu) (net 17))
 (segment (start 132.12 98.2) (end 132.12 101.04) (width 0.6) (layer B.Cu) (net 17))
 (segment (start 133.6 95.9) (end 134.65 96.95) (width 0.6) (layer B.Cu) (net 18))
 (segment (start 132.12 95.9) (end 133.6 95.9) (width 0.6) (layer B.Cu) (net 18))
 (segment (start 134.65 96.95) (end 134.65 101.05) (width 0.6) (layer B.Cu) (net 18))
 (segment (start 137.19 110.51) (end 136.4 111.3) (width 0.6) (layer B.Cu) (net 19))
 (segment (start 137.19 108.67) (end 137.19 110.51) (width 0.6) (layer B.Cu) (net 19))
 (segment (start 136.4 113) (end 137.25 113.85) (width 0.6) (layer B.Cu) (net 19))
 (segment (start 136.4 111.3) (end 136.4 113) (width 0.6) (layer B.Cu) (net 19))
 (segment (start 137.25 113.85) (end 140.75 113.85) (width 0.6) (layer B.Cu) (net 19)))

